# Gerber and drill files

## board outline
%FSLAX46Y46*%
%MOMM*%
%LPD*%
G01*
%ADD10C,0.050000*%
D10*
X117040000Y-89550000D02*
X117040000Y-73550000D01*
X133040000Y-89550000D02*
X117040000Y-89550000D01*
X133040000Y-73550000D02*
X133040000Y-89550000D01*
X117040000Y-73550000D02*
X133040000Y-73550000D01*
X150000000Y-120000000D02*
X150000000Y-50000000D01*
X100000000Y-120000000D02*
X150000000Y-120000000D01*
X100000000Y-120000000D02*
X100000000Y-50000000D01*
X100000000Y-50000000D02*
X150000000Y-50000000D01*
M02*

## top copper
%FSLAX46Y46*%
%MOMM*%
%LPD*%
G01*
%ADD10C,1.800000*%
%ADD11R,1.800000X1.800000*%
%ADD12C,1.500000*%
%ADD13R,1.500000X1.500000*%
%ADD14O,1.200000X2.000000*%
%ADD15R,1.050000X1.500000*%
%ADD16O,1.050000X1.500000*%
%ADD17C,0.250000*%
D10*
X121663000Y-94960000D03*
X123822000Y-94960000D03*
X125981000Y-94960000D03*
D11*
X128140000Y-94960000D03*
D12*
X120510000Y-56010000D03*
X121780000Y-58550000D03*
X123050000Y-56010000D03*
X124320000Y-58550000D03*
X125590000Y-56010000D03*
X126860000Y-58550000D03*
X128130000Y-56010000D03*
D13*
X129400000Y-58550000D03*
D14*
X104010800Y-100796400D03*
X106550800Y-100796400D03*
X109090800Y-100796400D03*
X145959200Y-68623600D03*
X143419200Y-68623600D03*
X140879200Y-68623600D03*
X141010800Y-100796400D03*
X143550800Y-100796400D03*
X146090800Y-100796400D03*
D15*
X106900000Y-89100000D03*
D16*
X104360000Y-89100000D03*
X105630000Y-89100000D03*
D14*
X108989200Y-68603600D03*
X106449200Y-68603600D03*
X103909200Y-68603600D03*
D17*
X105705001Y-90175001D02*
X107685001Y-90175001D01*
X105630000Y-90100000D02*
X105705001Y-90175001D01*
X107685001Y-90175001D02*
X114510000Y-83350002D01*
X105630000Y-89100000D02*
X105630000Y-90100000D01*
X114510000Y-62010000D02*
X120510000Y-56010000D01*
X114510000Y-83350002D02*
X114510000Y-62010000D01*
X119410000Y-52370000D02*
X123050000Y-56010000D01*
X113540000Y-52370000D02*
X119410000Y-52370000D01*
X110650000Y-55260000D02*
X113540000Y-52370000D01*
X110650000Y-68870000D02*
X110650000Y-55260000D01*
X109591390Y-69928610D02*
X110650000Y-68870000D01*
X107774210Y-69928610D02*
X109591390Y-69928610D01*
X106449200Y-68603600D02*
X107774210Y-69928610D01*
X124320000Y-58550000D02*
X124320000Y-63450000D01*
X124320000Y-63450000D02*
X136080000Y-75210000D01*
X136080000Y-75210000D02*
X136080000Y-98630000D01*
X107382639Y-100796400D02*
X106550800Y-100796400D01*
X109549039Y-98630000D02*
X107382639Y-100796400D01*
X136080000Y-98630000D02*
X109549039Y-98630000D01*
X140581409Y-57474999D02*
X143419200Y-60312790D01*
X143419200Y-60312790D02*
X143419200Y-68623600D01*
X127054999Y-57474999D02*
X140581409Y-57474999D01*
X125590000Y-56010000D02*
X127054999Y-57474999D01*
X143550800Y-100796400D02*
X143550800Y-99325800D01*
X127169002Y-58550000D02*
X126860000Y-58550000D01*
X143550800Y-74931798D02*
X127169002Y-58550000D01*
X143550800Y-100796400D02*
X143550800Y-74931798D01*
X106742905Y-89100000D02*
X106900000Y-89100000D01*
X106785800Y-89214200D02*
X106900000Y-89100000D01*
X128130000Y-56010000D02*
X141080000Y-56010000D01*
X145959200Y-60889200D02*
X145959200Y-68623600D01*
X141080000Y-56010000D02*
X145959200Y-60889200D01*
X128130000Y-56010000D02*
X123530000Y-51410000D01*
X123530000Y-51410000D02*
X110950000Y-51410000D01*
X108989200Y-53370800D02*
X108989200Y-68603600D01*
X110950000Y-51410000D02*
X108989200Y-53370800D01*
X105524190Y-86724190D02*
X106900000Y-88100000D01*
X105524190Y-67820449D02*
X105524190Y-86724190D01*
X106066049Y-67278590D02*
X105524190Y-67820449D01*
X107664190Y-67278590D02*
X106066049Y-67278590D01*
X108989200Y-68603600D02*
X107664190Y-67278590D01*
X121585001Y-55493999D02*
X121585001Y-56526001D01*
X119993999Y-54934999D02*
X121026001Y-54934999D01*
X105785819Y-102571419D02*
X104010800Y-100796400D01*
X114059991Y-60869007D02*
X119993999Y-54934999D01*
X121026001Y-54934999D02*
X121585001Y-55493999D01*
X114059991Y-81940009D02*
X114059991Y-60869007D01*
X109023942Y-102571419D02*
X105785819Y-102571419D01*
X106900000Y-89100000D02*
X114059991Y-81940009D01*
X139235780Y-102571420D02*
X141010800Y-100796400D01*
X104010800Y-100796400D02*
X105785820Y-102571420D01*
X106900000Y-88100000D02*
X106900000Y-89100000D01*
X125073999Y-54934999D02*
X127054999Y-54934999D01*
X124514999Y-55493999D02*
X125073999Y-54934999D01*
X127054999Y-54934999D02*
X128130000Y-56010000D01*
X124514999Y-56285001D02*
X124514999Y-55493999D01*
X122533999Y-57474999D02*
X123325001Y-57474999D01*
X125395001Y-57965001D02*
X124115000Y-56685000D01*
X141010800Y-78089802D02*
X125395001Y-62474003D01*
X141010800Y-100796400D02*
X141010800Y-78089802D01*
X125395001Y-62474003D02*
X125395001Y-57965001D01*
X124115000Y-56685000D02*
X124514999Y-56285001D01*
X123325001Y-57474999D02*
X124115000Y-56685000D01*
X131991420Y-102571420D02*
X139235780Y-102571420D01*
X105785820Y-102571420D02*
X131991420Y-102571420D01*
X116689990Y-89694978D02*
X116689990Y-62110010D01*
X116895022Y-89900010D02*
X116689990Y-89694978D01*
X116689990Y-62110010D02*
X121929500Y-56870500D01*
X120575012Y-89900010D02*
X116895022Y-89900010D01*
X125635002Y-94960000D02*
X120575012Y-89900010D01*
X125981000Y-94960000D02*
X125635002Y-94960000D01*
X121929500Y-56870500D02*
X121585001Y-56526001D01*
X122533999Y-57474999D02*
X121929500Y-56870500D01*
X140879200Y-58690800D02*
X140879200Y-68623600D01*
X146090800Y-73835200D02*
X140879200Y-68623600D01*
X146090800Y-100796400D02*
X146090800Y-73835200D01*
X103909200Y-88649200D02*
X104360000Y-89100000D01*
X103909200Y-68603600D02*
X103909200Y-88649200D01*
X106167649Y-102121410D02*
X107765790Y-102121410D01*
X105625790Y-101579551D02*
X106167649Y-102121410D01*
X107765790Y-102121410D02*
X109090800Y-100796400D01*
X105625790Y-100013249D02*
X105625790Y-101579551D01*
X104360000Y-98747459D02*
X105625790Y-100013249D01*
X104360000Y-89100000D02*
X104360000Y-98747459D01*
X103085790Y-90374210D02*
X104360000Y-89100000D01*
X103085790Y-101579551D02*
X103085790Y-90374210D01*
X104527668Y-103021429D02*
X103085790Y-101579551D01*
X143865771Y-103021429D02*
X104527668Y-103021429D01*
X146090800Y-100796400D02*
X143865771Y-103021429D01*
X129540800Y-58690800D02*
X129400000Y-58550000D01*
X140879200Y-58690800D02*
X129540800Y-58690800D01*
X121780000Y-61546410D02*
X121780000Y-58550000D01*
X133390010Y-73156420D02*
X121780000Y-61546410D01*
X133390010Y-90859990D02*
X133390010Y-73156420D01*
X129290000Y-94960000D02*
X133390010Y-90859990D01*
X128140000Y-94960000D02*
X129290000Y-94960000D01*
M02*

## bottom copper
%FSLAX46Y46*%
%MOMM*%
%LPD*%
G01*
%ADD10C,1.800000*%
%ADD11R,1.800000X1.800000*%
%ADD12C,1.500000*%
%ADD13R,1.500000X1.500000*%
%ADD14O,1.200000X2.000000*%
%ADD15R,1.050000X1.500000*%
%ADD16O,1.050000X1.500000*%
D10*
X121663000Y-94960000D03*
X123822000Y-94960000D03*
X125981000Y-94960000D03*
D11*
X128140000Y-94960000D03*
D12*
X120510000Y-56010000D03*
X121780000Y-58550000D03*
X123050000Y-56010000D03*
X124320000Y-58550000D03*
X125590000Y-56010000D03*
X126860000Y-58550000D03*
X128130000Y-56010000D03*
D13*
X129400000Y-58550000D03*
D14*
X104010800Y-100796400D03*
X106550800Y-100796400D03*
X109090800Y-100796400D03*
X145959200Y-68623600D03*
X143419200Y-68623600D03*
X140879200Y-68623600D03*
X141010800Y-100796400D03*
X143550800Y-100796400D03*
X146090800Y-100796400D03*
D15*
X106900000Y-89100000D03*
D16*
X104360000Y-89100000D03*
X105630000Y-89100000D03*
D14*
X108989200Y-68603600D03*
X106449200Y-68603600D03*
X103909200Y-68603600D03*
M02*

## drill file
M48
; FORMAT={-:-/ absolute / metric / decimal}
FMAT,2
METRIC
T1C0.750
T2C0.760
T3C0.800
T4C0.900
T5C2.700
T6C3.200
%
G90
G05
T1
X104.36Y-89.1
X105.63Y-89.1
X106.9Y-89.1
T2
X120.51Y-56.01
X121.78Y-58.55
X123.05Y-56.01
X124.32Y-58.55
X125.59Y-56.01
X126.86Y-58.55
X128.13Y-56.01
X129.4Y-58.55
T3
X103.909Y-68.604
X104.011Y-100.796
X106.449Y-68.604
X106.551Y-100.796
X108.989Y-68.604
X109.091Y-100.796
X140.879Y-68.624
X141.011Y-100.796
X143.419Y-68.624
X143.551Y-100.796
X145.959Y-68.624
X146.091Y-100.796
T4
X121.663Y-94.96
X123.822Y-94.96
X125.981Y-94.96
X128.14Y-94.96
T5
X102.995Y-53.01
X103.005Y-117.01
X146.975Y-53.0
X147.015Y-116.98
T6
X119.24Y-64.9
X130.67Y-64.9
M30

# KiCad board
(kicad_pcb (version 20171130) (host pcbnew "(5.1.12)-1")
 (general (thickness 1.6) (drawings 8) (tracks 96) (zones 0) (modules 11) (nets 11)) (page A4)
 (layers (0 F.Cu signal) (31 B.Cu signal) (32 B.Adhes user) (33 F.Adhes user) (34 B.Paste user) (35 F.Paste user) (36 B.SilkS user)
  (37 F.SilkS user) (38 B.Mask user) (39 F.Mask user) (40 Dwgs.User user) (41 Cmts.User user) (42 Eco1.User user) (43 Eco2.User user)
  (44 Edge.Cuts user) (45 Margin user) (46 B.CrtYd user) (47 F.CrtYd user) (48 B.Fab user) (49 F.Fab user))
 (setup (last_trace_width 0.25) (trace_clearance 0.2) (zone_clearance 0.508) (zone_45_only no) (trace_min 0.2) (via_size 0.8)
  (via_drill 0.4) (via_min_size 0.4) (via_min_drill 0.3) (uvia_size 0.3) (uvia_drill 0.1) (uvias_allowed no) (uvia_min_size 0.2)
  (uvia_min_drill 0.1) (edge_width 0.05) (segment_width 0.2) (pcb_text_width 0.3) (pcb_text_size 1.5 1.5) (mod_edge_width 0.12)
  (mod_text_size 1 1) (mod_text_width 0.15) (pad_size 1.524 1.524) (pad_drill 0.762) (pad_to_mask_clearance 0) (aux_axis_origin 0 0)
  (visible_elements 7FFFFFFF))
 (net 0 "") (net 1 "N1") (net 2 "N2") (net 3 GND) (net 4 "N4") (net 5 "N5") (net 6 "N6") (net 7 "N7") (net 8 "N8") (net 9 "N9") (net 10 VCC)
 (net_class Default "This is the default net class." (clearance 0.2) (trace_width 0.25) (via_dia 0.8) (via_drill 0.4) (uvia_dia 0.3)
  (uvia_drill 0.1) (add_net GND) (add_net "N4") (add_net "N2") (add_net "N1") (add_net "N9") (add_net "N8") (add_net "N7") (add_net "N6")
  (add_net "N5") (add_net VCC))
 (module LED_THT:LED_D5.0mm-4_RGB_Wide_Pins (layer F.Cu) (at 128.14 94.96 180)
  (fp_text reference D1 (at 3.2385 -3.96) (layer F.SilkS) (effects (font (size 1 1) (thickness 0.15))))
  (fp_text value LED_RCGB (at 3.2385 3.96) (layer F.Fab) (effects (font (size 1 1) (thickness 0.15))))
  (pad 4 thru_hole circle (at 6.477 0 180) (size 1.8 1.8) (drill 0.9) (layers *.Cu *.Mask) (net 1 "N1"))
  (pad 3 thru_hole circle (at 4.318 0 180) (size 1.8 1.8) (drill 0.9) (layers *.Cu *.Mask) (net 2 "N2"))
  (pad 2 thru_hole circle (at 2.159 0 180) (size 1.8 1.8) (drill 0.9) (layers *.Cu *.Mask) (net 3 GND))
  (pad 1 thru_hole rect (at 0 0 180) (size 1.8 1.8) (drill 0.9) (layers *.Cu *.Mask) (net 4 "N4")))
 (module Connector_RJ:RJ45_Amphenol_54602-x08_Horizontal (layer B.Cu) (at 129.4 58.55 180)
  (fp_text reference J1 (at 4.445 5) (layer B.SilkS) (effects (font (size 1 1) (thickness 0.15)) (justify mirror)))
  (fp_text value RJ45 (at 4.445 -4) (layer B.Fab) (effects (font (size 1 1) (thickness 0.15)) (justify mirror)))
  (pad 8 thru_hole circle (at 8.89 2.54 180) (size 1.5 1.5) (drill 0.76) (layers *.Cu *.Mask) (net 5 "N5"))
  (pad 7 thru_hole circle (at 7.62 0 180) (size 1.5 1.5) (drill 0.76) (layers *.Cu *.Mask) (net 4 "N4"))
  (pad 6 thru_hole circle (at 6.35 2.54 180) (size 1.5 1.5) (drill 0.76) (layers *.Cu *.Mask) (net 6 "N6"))
  (pad 5 thru_hole circle (at 5.08 0 180) (size 1.5 1.5) (drill 0.76) (layers *.Cu *.Mask) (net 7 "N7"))
  (pad 4 thru_hole circle (at 3.81 2.54 180) (size 1.5 1.5) (drill 0.76) (layers *.Cu *.Mask) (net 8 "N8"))
  (pad 3 thru_hole circle (at 2.54 0 180) (size 1.5 1.5) (drill 0.76) (layers *.Cu *.Mask) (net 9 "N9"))
  (pad 2 thru_hole circle (at 1.27 2.54 180) (size 1.5 1.5) (drill 0.76) (layers *.Cu *.Mask) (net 3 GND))
  (pad 1 thru_hole rect (at 0 0 180) (size 1.5 1.5) (drill 0.76) (layers *.Cu *.Mask) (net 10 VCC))
  (pad "" np_thru_hole circle (at -1.27 -6.35 180) (size 3.2 3.2) (drill 3.2) (layers *.Cu *.Mask))
  (pad "" np_thru_hole circle (at 10.16 -6.35 180) (size 3.2 3.2) (drill 3.2) (layers *.Cu *.Mask)))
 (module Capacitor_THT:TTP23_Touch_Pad (layer F.Cu) (at 106.5 104.2)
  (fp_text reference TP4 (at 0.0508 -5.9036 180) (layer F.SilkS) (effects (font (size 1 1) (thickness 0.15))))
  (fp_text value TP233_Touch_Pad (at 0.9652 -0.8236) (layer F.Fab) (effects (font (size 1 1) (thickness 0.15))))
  (pad 3 thru_hole oval (at -2.4892 -3.4036 180) (size 1.2 2) (drill 0.8) (layers *.Cu *.Mask) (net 3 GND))
  (pad 2 thru_hole oval (at 0.0508 -3.4036 180) (size 1.2 2) (drill 0.8) (layers *.Cu *.Mask) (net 7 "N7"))
  (pad 1 thru_hole oval (at 2.5908 -3.4036 180) (size 1.2 2) (drill 0.8) (layers *.Cu *.Mask) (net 10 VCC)))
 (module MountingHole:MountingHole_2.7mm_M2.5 (layer F.Cu) (at 146.975 53)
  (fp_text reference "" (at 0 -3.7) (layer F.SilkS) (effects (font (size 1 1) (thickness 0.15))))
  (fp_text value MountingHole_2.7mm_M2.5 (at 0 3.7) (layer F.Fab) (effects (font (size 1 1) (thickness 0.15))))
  (pad 1 np_thru_hole circle (at 0 0) (size 2.7 2.7) (drill 2.7) (layers *.Cu *.Mask)))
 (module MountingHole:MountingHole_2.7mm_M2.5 (layer F.Cu) (at 147.015 116.98)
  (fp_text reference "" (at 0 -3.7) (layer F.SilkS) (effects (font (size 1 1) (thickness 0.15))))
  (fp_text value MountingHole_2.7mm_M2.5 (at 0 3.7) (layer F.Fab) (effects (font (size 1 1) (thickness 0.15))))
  (pad 1 np_thru_hole circle (at 0 0) (size 2.7 2.7) (drill 2.7) (layers *.Cu *.Mask)))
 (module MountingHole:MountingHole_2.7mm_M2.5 (layer F.Cu) (at 103.005 117.01)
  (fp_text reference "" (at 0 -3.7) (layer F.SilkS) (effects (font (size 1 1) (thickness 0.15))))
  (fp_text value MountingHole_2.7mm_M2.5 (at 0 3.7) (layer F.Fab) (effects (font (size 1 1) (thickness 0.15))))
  (pad 1 np_thru_hole circle (at 0 0) (size 2.7 2.7) (drill 2.7) (layers *.Cu *.Mask)))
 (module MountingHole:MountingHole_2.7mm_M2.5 (layer F.Cu) (at 102.995 53.01)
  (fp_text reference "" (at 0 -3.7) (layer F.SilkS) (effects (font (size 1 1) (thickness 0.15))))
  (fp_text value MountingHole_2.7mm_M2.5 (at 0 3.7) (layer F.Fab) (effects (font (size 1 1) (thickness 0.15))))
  (pad 1 np_thru_hole circle (at 0 0) (size 2.7 2.7) (drill 2.7) (layers *.Cu *.Mask)))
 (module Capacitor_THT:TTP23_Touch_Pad (layer F.Cu) (at 143.47 65.22 180)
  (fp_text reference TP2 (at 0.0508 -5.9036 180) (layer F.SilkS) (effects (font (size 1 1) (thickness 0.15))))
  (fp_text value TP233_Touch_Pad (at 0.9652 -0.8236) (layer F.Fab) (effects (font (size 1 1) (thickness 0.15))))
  (pad 3 thru_hole oval (at -2.4892 -3.4036) (size 1.2 2) (drill 0.8) (layers *.Cu *.Mask) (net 3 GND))
  (pad 2 thru_hole oval (at 0.0508 -3.4036) (size 1.2 2) (drill 0.8) (layers *.Cu *.Mask) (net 8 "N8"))
  (pad 1 thru_hole oval (at 2.5908 -3.4036) (size 1.2 2) (drill 0.8) (layers *.Cu *.Mask) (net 10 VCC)))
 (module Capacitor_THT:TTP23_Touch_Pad (layer F.Cu) (at 143.5 104.2)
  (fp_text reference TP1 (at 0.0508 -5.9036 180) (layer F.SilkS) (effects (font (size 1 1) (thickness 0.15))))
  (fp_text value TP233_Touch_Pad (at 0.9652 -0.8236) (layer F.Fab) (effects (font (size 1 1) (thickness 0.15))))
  (pad 3 thru_hole oval (at -2.4892 -3.4036 180) (size 1.2 2) (drill 0.8) (layers *.Cu *.Mask) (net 3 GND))
  (pad 2 thru_hole oval (at 0.0508 -3.4036 180) (size 1.2 2) (drill 0.8) (layers *.Cu *.Mask) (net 9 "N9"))
  (pad 1 thru_hole oval (at 2.5908 -3.4036 180) (size 1.2 2) (drill 0.8) (layers *.Cu *.Mask) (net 10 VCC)))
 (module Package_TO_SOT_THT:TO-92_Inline (layer F.Cu) (at 106.9 89.1 180)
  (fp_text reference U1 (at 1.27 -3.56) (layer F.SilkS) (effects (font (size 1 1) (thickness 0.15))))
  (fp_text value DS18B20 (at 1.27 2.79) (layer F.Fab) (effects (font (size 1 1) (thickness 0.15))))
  (pad 1 thru_hole rect (at 0 0 180) (size 1.05 1.5) (drill 0.75) (layers *.Cu *.Mask) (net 3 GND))
  (pad 3 thru_hole oval (at 2.54 0 180) (size 1.05 1.5) (drill 0.75) (layers *.Cu *.Mask) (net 10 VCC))
  (pad 2 thru_hole oval (at 1.27 0 180) (size 1.05 1.5) (drill 0.75) (layers *.Cu *.Mask) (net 5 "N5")))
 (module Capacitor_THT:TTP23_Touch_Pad (layer F.Cu) (at 106.5 65.2 180)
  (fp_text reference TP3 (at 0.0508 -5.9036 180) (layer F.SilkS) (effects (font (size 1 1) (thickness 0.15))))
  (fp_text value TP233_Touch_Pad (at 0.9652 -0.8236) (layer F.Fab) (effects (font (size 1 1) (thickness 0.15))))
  (pad 3 thru_hole oval (at -2.4892 -3.4036) (size 1.2 2) (drill 0.8) (layers *.Cu *.Mask) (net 3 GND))
  (pad 2 thru_hole oval (at 0.0508 -3.4036) (size 1.2 2) (drill 0.8) (layers *.Cu *.Mask) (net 6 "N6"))
  (pad 1 thru_hole oval (at 2.5908 -3.4036) (size 1.2 2) (drill 0.8) (layers *.Cu *.Mask) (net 10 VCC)))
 (gr_line (start 117.04 89.55) (end 117.04 73.55) (layer Edge.Cuts) (width 0.05))
 (gr_line (start 133.04 89.55) (end 117.04 89.55) (layer Edge.Cuts) (width 0.05))
 (gr_line (start 133.04 73.55) (end 133.04 89.55) (layer Edge.Cuts) (width 0.05))
 (gr_line (start 117.04 73.55) (end 133.04 73.55) (layer Edge.Cuts) (width 0.05))
 (gr_line (start 150 120) (end 150 50) (layer Edge.Cuts) (width 0.05))
 (gr_line (start 100 120) (end 150 120) (layer Edge.Cuts) (width 0.05))
 (gr_line (start 100 120) (end 100 50) (layer Edge.Cuts) (width 0.05))
 (gr_line (start 100 50) (end 150 50) (layer Edge.Cuts) (width 0.05))
 (segment (start 105.705001 90.175001) (end 107.685001 90.175001) (width 0.25) (layer F.Cu) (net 5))
 (segment (start 105.63 90.1) (end 105.705001 90.175001) (width 0.25) (layer F.Cu) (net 5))
 (segment (start 107.685001 90.175001) (end 114.51 83.350002) (width 0.25) (layer F.Cu) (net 5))
 (segment (start 105.63 89.1) (end 105.63 90.1) (width 0.25) (layer F.Cu) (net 5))
 (segment (start 114.51 62.01) (end 120.51 56.01) (width 0.25) (layer F.Cu) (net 5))
 (segment (start 114.51 83.350002) (end 114.51 62.01) (width 0.25) (layer F.Cu) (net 5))
 (segment (start 119.41 52.37) (end 123.05 56.01) (width 0.25) (layer F.Cu) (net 6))
 (segment (start 113.54 52.37) (end 119.41 52.37) (width 0.25) (layer F.Cu) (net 6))
 (segment (start 110.65 55.26) (end 113.54 52.37) (width 0.25) (layer F.Cu) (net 6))
 (segment (start 110.65 68.87) (end 110.65 55.26) (width 0.25) (layer F.Cu) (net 6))
 (segment (start 109.59139 69.92861) (end 110.65 68.87) (width 0.25) (layer F.Cu) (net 6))
 (segment (start 107.77421 69.92861) (end 109.59139 69.92861) (width 0.25) (layer F.Cu) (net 6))
 (segment (start 106.4492 68.6036) (end 107.77421 69.92861) (width 0.25) (layer F.Cu) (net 6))
 (segment (start 124.32 58.55) (end 124.32 63.45) (width 0.25) (layer F.Cu) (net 7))
 (segment (start 124.32 63.45) (end 136.08 75.21) (width 0.25) (layer F.Cu) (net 7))
 (segment (start 136.08 75.21) (end 136.08 98.63) (width 0.25) (layer F.Cu) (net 7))
 (segment (start 107.382639 100.7964) (end 106.5508 100.7964) (width 0.25) (layer F.Cu) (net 7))
 (segment (start 109.549039 98.63) (end 107.382639 100.7964) (width 0.25) (layer F.Cu) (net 7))
 (segment (start 136.08 98.63) (end 109.549039 98.63) (width 0.25) (layer F.Cu) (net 7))
 (segment (start 140.581409 57.474999) (end 143.4192 60.31279) (width 0.25) (layer F.Cu) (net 8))
 (segment (start 143.4192 60.31279) (end 143.4192 68.6236) (width 0.25) (layer F.Cu) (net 8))
 (segment (start 127.054999 57.474999) (end 140.581409 57.474999) (width 0.25) (layer F.Cu) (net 8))
 (segment (start 125.59 56.01) (end 127.054999 57.474999) (width 0.25) (layer F.Cu) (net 8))
 (segment (start 143.5508 100.7964) (end 143.5508 99.3258) (width 0.25) (layer F.Cu) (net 9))
 (segment (start 127.169002 58.55) (end 126.86 58.55) (width 0.25) (layer F.Cu) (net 9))
 (segment (start 143.5508 74.931798) (end 127.169002 58.55) (width 0.25) (layer F.Cu) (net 9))
 (segment (start 143.5508 100.7964) (end 143.5508 74.931798) (width 0.25) (layer F.Cu) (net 9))
 (segment (start 106.742905 89.1) (end 106.9 89.1) (width 0.25) (layer F.Cu) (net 3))
 (segment (start 106.7858 89.2142) (end 106.9 89.1) (width 0.25) (layer F.Cu) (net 3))
 (segment (start 128.13 56.01) (end 141.08 56.01) (width 0.25) (layer F.Cu) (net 3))
 (segment (start 145.9592 60.8892) (end 145.9592 68.6236) (width 0.25) (layer F.Cu) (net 3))
 (segment (start 141.08 56.01) (end 145.9592 60.8892) (width 0.25) (layer F.Cu) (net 3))
 (segment (start 128.13 56.01) (end 123.53 51.41) (width 0.25) (layer F.Cu) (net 3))
 (segment (start 123.53 51.41) (end 110.95 51.41) (width 0.25) (layer F.Cu) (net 3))
 (segment (start 108.9892 53.3708) (end 108.9892 68.6036) (width 0.25) (layer F.Cu) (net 3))
 (segment (start 110.95 51.41) (end 108.9892 53.3708) (width 0.25) (layer F.Cu) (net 3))
 (segment (start 105.52419 86.72419) (end 106.9 88.1) (width 0.25) (layer F.Cu) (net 3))
 (segment (start 105.52419 67.820449) (end 105.52419 86.72419) (width 0.25) (layer F.Cu) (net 3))
 (segment (start 106.066049 67.27859) (end 105.52419 67.820449) (width 0.25) (layer F.Cu) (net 3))
 (segment (start 107.66419 67.27859) (end 106.066049 67.27859) (width 0.25) (layer F.Cu) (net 3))
 (segment (start 108.9892 68.6036) (end 107.66419 67.27859) (width 0.25) (layer F.Cu) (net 3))
 (segment (start 121.585001 55.493999) (end 121.585001 56.526001) (width 0.25) (layer F.Cu) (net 3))
 (segment (start 119.993999 54.934999) (end 121.026001 54.934999) (width 0.25) (layer F.Cu) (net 3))
 (segment (start 105.785819 102.571419) (end 104.0108 100.7964) (width 0.25) (layer F.Cu) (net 3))
 (segment (start 114.059991 60.869007) (end 119.993999 54.934999) (width 0.25) (layer F.Cu) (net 3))
 (segment (start 121.026001 54.934999) (end 121.585001 55.493999) (width 0.25) (layer F.Cu) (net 3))
 (segment (start 114.059991 81.940009) (end 114.059991 60.869007) (width 0.25) (layer F.Cu) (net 3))
 (segment (start 109.023942 102.571419) (end 105.785819 102.571419) (width 0.25) (layer F.Cu) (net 3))
 (segment (start 106.9 89.1) (end 114.059991 81.940009) (width 0.25) (layer F.Cu) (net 3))
 (segment (start 139.23578 102.57142) (end 141.0108 100.7964) (width 0.25) (layer F.Cu) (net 3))
 (segment (start 104.0108 100.7964) (end 105.78582 102.57142) (width 0.25) (layer F.Cu) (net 3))
 (segment (start 106.9 88.1) (end 106.9 89.1) (width 0.25) (layer F.Cu) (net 3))
 (segment (start 125.073999 54.934999) (end 127.054999 54.934999) (width 0.25) (layer F.Cu) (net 3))
 (segment (start 124.514999 55.493999) (end 125.073999 54.934999) (width 0.25) (layer F.Cu) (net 3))
 (segment (start 127.054999 54.934999) (end 128.13 56.01) (width 0.25) (layer F.Cu) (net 3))
 (segment (start 124.514999 56.285001) (end 124.514999 55.493999) (width 0.25) (layer F.Cu) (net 3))
 (segment (start 122.533999 57.474999) (end 123.325001 57.474999) (width 0.25) (layer F.Cu) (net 3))
 (segment (start 125.395001 57.965001) (end 124.115 56.685) (width 0.25) (layer F.Cu) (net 3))
 (segment (start 141.0108 78.089802) (end 125.395001 62.474003) (width 0.25) (layer F.Cu) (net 3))
 (segment (start 141.0108 100.7964) (end 141.0108 78.089802) (width 0.25) (layer F.Cu) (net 3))
 (segment (start 125.395001 62.474003) (end 125.395001 57.965001) (width 0.25) (layer F.Cu) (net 3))
 (segment (start 124.115 56.685) (end 124.514999 56.285001) (width 0.25) (layer F.Cu) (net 3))
 (segment (start 123.325001 57.474999) (end 124.115 56.685) (width 0.25) (layer F.Cu) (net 3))
 (segment (start 131.99142 102.57142) (end 139.23578 102.57142) (width 0.25) (layer F.Cu) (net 3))
 (segment (start 105.78582 102.57142) (end 131.99142 102.57142) (width 0.25) (layer F.Cu) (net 3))
 (segment (start 116.68999 89.694978) (end 116.68999 62.11001) (width 0.25) (layer F.Cu) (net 3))
 (segment (start 116.895022 89.90001) (end 116.68999 89.694978) (width 0.25) (layer F.Cu) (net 3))
 (segment (start 116.68999 62.11001) (end 121.9295 56.8705) (width 0.25) (layer F.Cu) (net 3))
 (segment (start 120.575012 89.90001) (end 116.895022 89.90001) (width 0.25) (layer F.Cu) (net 3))
 (segment (start 125.635002 94.96) (end 120.575012 89.90001) (width 0.25) (layer F.Cu) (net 3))
 (segment (start 125.981 94.96) (end 125.635002 94.96) (width 0.25) (layer F.Cu) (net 3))
 (segment (start 121.9295 56.8705) (end 121.585001 56.526001) (width 0.25) (layer F.Cu) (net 3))
 (segment (start 122.533999 57.474999) (end 121.9295 56.8705) (width 0.25) (layer F.Cu) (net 3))
 (segment (start 140.8792 58.6908) (end 140.8792 68.6236) (width 0.25) (layer F.Cu) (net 10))
 (segment (start 146.0908 73.8352) (end 140.8792 68.6236) (width 0.25) (layer F.Cu) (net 10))
 (segment (start 146.0908 100.7964) (end 146.0908 73.8352) (width 0.25) (layer F.Cu) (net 10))
 (segment (start 103.9092 88.6492) (end 104.36 89.1) (width 0.25) (layer F.Cu) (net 10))
 (segment (start 103.9092 68.6036) (end 103.9092 88.6492) (width 0.25) (layer F.Cu) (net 10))
 (segment (start 106.167649 102.12141) (end 107.76579 102.12141) (width 0.25) (layer F.Cu) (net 10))
 (segment (start 105.62579 101.579551) (end 106.167649 102.12141) (width 0.25) (layer F.Cu) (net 10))
 (segment (start 107.76579 102.12141) (end 109.0908 100.7964) (width 0.25) (layer F.Cu) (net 10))
 (segment (start 105.62579 100.013249) (end 105.62579 101.579551) (width 0.25) (layer F.Cu) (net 10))
 (segment (start 104.36 98.747459) (end 105.62579 100.013249) (width 0.25) (layer F.Cu) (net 10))
 (segment (start 104.36 89.1) (end 104.36 98.747459) (width 0.25) (layer F.Cu) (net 10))
 (segment (start 103.08579 90.37421) (end 104.36 89.1) (width 0.25) (layer F.Cu) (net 10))
 (segment (start 103.08579 101.579551) (end 103.08579 90.37421) (width 0.25) (layer F.Cu) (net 10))
 (segment (start 104.527668 103.021429) (end 103.08579 101.579551) (width 0.25) (layer F.Cu) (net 10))
 (segment (start 143.865771 103.021429) (end 104.527668 103.021429) (width 0.25) (layer F.Cu) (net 10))
 (segment (start 146.0908 100.7964) (end 143.865771 103.021429) (width 0.25) (layer F.Cu) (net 10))
 (segment (start 129.5408 58.6908) (end 129.4 58.55) (width 0.25) (layer F.Cu) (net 10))
 (segment (start 140.8792 58.6908) (end 129.5408 58.6908) (width 0.25) (layer F.Cu) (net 10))
 (segment (start 121.78 61.54641) (end 121.78 58.55) (width 0.25) (layer F.Cu) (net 4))
 (segment (start 133.39001 73.15642) (end 121.78 61.54641) (width 0.25) (layer F.Cu) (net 4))
 (segment (start 133.39001 90.85999) (end 133.39001 73.15642) (width 0.25) (layer F.Cu) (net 4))
 (segment (start 129.29 94.96) (end 133.39001 90.85999) (width 0.25) (layer F.Cu) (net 4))
 (segment (start 128.14 94.96) (end 129.29 94.96) (width 0.25) (layer F.Cu) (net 4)))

